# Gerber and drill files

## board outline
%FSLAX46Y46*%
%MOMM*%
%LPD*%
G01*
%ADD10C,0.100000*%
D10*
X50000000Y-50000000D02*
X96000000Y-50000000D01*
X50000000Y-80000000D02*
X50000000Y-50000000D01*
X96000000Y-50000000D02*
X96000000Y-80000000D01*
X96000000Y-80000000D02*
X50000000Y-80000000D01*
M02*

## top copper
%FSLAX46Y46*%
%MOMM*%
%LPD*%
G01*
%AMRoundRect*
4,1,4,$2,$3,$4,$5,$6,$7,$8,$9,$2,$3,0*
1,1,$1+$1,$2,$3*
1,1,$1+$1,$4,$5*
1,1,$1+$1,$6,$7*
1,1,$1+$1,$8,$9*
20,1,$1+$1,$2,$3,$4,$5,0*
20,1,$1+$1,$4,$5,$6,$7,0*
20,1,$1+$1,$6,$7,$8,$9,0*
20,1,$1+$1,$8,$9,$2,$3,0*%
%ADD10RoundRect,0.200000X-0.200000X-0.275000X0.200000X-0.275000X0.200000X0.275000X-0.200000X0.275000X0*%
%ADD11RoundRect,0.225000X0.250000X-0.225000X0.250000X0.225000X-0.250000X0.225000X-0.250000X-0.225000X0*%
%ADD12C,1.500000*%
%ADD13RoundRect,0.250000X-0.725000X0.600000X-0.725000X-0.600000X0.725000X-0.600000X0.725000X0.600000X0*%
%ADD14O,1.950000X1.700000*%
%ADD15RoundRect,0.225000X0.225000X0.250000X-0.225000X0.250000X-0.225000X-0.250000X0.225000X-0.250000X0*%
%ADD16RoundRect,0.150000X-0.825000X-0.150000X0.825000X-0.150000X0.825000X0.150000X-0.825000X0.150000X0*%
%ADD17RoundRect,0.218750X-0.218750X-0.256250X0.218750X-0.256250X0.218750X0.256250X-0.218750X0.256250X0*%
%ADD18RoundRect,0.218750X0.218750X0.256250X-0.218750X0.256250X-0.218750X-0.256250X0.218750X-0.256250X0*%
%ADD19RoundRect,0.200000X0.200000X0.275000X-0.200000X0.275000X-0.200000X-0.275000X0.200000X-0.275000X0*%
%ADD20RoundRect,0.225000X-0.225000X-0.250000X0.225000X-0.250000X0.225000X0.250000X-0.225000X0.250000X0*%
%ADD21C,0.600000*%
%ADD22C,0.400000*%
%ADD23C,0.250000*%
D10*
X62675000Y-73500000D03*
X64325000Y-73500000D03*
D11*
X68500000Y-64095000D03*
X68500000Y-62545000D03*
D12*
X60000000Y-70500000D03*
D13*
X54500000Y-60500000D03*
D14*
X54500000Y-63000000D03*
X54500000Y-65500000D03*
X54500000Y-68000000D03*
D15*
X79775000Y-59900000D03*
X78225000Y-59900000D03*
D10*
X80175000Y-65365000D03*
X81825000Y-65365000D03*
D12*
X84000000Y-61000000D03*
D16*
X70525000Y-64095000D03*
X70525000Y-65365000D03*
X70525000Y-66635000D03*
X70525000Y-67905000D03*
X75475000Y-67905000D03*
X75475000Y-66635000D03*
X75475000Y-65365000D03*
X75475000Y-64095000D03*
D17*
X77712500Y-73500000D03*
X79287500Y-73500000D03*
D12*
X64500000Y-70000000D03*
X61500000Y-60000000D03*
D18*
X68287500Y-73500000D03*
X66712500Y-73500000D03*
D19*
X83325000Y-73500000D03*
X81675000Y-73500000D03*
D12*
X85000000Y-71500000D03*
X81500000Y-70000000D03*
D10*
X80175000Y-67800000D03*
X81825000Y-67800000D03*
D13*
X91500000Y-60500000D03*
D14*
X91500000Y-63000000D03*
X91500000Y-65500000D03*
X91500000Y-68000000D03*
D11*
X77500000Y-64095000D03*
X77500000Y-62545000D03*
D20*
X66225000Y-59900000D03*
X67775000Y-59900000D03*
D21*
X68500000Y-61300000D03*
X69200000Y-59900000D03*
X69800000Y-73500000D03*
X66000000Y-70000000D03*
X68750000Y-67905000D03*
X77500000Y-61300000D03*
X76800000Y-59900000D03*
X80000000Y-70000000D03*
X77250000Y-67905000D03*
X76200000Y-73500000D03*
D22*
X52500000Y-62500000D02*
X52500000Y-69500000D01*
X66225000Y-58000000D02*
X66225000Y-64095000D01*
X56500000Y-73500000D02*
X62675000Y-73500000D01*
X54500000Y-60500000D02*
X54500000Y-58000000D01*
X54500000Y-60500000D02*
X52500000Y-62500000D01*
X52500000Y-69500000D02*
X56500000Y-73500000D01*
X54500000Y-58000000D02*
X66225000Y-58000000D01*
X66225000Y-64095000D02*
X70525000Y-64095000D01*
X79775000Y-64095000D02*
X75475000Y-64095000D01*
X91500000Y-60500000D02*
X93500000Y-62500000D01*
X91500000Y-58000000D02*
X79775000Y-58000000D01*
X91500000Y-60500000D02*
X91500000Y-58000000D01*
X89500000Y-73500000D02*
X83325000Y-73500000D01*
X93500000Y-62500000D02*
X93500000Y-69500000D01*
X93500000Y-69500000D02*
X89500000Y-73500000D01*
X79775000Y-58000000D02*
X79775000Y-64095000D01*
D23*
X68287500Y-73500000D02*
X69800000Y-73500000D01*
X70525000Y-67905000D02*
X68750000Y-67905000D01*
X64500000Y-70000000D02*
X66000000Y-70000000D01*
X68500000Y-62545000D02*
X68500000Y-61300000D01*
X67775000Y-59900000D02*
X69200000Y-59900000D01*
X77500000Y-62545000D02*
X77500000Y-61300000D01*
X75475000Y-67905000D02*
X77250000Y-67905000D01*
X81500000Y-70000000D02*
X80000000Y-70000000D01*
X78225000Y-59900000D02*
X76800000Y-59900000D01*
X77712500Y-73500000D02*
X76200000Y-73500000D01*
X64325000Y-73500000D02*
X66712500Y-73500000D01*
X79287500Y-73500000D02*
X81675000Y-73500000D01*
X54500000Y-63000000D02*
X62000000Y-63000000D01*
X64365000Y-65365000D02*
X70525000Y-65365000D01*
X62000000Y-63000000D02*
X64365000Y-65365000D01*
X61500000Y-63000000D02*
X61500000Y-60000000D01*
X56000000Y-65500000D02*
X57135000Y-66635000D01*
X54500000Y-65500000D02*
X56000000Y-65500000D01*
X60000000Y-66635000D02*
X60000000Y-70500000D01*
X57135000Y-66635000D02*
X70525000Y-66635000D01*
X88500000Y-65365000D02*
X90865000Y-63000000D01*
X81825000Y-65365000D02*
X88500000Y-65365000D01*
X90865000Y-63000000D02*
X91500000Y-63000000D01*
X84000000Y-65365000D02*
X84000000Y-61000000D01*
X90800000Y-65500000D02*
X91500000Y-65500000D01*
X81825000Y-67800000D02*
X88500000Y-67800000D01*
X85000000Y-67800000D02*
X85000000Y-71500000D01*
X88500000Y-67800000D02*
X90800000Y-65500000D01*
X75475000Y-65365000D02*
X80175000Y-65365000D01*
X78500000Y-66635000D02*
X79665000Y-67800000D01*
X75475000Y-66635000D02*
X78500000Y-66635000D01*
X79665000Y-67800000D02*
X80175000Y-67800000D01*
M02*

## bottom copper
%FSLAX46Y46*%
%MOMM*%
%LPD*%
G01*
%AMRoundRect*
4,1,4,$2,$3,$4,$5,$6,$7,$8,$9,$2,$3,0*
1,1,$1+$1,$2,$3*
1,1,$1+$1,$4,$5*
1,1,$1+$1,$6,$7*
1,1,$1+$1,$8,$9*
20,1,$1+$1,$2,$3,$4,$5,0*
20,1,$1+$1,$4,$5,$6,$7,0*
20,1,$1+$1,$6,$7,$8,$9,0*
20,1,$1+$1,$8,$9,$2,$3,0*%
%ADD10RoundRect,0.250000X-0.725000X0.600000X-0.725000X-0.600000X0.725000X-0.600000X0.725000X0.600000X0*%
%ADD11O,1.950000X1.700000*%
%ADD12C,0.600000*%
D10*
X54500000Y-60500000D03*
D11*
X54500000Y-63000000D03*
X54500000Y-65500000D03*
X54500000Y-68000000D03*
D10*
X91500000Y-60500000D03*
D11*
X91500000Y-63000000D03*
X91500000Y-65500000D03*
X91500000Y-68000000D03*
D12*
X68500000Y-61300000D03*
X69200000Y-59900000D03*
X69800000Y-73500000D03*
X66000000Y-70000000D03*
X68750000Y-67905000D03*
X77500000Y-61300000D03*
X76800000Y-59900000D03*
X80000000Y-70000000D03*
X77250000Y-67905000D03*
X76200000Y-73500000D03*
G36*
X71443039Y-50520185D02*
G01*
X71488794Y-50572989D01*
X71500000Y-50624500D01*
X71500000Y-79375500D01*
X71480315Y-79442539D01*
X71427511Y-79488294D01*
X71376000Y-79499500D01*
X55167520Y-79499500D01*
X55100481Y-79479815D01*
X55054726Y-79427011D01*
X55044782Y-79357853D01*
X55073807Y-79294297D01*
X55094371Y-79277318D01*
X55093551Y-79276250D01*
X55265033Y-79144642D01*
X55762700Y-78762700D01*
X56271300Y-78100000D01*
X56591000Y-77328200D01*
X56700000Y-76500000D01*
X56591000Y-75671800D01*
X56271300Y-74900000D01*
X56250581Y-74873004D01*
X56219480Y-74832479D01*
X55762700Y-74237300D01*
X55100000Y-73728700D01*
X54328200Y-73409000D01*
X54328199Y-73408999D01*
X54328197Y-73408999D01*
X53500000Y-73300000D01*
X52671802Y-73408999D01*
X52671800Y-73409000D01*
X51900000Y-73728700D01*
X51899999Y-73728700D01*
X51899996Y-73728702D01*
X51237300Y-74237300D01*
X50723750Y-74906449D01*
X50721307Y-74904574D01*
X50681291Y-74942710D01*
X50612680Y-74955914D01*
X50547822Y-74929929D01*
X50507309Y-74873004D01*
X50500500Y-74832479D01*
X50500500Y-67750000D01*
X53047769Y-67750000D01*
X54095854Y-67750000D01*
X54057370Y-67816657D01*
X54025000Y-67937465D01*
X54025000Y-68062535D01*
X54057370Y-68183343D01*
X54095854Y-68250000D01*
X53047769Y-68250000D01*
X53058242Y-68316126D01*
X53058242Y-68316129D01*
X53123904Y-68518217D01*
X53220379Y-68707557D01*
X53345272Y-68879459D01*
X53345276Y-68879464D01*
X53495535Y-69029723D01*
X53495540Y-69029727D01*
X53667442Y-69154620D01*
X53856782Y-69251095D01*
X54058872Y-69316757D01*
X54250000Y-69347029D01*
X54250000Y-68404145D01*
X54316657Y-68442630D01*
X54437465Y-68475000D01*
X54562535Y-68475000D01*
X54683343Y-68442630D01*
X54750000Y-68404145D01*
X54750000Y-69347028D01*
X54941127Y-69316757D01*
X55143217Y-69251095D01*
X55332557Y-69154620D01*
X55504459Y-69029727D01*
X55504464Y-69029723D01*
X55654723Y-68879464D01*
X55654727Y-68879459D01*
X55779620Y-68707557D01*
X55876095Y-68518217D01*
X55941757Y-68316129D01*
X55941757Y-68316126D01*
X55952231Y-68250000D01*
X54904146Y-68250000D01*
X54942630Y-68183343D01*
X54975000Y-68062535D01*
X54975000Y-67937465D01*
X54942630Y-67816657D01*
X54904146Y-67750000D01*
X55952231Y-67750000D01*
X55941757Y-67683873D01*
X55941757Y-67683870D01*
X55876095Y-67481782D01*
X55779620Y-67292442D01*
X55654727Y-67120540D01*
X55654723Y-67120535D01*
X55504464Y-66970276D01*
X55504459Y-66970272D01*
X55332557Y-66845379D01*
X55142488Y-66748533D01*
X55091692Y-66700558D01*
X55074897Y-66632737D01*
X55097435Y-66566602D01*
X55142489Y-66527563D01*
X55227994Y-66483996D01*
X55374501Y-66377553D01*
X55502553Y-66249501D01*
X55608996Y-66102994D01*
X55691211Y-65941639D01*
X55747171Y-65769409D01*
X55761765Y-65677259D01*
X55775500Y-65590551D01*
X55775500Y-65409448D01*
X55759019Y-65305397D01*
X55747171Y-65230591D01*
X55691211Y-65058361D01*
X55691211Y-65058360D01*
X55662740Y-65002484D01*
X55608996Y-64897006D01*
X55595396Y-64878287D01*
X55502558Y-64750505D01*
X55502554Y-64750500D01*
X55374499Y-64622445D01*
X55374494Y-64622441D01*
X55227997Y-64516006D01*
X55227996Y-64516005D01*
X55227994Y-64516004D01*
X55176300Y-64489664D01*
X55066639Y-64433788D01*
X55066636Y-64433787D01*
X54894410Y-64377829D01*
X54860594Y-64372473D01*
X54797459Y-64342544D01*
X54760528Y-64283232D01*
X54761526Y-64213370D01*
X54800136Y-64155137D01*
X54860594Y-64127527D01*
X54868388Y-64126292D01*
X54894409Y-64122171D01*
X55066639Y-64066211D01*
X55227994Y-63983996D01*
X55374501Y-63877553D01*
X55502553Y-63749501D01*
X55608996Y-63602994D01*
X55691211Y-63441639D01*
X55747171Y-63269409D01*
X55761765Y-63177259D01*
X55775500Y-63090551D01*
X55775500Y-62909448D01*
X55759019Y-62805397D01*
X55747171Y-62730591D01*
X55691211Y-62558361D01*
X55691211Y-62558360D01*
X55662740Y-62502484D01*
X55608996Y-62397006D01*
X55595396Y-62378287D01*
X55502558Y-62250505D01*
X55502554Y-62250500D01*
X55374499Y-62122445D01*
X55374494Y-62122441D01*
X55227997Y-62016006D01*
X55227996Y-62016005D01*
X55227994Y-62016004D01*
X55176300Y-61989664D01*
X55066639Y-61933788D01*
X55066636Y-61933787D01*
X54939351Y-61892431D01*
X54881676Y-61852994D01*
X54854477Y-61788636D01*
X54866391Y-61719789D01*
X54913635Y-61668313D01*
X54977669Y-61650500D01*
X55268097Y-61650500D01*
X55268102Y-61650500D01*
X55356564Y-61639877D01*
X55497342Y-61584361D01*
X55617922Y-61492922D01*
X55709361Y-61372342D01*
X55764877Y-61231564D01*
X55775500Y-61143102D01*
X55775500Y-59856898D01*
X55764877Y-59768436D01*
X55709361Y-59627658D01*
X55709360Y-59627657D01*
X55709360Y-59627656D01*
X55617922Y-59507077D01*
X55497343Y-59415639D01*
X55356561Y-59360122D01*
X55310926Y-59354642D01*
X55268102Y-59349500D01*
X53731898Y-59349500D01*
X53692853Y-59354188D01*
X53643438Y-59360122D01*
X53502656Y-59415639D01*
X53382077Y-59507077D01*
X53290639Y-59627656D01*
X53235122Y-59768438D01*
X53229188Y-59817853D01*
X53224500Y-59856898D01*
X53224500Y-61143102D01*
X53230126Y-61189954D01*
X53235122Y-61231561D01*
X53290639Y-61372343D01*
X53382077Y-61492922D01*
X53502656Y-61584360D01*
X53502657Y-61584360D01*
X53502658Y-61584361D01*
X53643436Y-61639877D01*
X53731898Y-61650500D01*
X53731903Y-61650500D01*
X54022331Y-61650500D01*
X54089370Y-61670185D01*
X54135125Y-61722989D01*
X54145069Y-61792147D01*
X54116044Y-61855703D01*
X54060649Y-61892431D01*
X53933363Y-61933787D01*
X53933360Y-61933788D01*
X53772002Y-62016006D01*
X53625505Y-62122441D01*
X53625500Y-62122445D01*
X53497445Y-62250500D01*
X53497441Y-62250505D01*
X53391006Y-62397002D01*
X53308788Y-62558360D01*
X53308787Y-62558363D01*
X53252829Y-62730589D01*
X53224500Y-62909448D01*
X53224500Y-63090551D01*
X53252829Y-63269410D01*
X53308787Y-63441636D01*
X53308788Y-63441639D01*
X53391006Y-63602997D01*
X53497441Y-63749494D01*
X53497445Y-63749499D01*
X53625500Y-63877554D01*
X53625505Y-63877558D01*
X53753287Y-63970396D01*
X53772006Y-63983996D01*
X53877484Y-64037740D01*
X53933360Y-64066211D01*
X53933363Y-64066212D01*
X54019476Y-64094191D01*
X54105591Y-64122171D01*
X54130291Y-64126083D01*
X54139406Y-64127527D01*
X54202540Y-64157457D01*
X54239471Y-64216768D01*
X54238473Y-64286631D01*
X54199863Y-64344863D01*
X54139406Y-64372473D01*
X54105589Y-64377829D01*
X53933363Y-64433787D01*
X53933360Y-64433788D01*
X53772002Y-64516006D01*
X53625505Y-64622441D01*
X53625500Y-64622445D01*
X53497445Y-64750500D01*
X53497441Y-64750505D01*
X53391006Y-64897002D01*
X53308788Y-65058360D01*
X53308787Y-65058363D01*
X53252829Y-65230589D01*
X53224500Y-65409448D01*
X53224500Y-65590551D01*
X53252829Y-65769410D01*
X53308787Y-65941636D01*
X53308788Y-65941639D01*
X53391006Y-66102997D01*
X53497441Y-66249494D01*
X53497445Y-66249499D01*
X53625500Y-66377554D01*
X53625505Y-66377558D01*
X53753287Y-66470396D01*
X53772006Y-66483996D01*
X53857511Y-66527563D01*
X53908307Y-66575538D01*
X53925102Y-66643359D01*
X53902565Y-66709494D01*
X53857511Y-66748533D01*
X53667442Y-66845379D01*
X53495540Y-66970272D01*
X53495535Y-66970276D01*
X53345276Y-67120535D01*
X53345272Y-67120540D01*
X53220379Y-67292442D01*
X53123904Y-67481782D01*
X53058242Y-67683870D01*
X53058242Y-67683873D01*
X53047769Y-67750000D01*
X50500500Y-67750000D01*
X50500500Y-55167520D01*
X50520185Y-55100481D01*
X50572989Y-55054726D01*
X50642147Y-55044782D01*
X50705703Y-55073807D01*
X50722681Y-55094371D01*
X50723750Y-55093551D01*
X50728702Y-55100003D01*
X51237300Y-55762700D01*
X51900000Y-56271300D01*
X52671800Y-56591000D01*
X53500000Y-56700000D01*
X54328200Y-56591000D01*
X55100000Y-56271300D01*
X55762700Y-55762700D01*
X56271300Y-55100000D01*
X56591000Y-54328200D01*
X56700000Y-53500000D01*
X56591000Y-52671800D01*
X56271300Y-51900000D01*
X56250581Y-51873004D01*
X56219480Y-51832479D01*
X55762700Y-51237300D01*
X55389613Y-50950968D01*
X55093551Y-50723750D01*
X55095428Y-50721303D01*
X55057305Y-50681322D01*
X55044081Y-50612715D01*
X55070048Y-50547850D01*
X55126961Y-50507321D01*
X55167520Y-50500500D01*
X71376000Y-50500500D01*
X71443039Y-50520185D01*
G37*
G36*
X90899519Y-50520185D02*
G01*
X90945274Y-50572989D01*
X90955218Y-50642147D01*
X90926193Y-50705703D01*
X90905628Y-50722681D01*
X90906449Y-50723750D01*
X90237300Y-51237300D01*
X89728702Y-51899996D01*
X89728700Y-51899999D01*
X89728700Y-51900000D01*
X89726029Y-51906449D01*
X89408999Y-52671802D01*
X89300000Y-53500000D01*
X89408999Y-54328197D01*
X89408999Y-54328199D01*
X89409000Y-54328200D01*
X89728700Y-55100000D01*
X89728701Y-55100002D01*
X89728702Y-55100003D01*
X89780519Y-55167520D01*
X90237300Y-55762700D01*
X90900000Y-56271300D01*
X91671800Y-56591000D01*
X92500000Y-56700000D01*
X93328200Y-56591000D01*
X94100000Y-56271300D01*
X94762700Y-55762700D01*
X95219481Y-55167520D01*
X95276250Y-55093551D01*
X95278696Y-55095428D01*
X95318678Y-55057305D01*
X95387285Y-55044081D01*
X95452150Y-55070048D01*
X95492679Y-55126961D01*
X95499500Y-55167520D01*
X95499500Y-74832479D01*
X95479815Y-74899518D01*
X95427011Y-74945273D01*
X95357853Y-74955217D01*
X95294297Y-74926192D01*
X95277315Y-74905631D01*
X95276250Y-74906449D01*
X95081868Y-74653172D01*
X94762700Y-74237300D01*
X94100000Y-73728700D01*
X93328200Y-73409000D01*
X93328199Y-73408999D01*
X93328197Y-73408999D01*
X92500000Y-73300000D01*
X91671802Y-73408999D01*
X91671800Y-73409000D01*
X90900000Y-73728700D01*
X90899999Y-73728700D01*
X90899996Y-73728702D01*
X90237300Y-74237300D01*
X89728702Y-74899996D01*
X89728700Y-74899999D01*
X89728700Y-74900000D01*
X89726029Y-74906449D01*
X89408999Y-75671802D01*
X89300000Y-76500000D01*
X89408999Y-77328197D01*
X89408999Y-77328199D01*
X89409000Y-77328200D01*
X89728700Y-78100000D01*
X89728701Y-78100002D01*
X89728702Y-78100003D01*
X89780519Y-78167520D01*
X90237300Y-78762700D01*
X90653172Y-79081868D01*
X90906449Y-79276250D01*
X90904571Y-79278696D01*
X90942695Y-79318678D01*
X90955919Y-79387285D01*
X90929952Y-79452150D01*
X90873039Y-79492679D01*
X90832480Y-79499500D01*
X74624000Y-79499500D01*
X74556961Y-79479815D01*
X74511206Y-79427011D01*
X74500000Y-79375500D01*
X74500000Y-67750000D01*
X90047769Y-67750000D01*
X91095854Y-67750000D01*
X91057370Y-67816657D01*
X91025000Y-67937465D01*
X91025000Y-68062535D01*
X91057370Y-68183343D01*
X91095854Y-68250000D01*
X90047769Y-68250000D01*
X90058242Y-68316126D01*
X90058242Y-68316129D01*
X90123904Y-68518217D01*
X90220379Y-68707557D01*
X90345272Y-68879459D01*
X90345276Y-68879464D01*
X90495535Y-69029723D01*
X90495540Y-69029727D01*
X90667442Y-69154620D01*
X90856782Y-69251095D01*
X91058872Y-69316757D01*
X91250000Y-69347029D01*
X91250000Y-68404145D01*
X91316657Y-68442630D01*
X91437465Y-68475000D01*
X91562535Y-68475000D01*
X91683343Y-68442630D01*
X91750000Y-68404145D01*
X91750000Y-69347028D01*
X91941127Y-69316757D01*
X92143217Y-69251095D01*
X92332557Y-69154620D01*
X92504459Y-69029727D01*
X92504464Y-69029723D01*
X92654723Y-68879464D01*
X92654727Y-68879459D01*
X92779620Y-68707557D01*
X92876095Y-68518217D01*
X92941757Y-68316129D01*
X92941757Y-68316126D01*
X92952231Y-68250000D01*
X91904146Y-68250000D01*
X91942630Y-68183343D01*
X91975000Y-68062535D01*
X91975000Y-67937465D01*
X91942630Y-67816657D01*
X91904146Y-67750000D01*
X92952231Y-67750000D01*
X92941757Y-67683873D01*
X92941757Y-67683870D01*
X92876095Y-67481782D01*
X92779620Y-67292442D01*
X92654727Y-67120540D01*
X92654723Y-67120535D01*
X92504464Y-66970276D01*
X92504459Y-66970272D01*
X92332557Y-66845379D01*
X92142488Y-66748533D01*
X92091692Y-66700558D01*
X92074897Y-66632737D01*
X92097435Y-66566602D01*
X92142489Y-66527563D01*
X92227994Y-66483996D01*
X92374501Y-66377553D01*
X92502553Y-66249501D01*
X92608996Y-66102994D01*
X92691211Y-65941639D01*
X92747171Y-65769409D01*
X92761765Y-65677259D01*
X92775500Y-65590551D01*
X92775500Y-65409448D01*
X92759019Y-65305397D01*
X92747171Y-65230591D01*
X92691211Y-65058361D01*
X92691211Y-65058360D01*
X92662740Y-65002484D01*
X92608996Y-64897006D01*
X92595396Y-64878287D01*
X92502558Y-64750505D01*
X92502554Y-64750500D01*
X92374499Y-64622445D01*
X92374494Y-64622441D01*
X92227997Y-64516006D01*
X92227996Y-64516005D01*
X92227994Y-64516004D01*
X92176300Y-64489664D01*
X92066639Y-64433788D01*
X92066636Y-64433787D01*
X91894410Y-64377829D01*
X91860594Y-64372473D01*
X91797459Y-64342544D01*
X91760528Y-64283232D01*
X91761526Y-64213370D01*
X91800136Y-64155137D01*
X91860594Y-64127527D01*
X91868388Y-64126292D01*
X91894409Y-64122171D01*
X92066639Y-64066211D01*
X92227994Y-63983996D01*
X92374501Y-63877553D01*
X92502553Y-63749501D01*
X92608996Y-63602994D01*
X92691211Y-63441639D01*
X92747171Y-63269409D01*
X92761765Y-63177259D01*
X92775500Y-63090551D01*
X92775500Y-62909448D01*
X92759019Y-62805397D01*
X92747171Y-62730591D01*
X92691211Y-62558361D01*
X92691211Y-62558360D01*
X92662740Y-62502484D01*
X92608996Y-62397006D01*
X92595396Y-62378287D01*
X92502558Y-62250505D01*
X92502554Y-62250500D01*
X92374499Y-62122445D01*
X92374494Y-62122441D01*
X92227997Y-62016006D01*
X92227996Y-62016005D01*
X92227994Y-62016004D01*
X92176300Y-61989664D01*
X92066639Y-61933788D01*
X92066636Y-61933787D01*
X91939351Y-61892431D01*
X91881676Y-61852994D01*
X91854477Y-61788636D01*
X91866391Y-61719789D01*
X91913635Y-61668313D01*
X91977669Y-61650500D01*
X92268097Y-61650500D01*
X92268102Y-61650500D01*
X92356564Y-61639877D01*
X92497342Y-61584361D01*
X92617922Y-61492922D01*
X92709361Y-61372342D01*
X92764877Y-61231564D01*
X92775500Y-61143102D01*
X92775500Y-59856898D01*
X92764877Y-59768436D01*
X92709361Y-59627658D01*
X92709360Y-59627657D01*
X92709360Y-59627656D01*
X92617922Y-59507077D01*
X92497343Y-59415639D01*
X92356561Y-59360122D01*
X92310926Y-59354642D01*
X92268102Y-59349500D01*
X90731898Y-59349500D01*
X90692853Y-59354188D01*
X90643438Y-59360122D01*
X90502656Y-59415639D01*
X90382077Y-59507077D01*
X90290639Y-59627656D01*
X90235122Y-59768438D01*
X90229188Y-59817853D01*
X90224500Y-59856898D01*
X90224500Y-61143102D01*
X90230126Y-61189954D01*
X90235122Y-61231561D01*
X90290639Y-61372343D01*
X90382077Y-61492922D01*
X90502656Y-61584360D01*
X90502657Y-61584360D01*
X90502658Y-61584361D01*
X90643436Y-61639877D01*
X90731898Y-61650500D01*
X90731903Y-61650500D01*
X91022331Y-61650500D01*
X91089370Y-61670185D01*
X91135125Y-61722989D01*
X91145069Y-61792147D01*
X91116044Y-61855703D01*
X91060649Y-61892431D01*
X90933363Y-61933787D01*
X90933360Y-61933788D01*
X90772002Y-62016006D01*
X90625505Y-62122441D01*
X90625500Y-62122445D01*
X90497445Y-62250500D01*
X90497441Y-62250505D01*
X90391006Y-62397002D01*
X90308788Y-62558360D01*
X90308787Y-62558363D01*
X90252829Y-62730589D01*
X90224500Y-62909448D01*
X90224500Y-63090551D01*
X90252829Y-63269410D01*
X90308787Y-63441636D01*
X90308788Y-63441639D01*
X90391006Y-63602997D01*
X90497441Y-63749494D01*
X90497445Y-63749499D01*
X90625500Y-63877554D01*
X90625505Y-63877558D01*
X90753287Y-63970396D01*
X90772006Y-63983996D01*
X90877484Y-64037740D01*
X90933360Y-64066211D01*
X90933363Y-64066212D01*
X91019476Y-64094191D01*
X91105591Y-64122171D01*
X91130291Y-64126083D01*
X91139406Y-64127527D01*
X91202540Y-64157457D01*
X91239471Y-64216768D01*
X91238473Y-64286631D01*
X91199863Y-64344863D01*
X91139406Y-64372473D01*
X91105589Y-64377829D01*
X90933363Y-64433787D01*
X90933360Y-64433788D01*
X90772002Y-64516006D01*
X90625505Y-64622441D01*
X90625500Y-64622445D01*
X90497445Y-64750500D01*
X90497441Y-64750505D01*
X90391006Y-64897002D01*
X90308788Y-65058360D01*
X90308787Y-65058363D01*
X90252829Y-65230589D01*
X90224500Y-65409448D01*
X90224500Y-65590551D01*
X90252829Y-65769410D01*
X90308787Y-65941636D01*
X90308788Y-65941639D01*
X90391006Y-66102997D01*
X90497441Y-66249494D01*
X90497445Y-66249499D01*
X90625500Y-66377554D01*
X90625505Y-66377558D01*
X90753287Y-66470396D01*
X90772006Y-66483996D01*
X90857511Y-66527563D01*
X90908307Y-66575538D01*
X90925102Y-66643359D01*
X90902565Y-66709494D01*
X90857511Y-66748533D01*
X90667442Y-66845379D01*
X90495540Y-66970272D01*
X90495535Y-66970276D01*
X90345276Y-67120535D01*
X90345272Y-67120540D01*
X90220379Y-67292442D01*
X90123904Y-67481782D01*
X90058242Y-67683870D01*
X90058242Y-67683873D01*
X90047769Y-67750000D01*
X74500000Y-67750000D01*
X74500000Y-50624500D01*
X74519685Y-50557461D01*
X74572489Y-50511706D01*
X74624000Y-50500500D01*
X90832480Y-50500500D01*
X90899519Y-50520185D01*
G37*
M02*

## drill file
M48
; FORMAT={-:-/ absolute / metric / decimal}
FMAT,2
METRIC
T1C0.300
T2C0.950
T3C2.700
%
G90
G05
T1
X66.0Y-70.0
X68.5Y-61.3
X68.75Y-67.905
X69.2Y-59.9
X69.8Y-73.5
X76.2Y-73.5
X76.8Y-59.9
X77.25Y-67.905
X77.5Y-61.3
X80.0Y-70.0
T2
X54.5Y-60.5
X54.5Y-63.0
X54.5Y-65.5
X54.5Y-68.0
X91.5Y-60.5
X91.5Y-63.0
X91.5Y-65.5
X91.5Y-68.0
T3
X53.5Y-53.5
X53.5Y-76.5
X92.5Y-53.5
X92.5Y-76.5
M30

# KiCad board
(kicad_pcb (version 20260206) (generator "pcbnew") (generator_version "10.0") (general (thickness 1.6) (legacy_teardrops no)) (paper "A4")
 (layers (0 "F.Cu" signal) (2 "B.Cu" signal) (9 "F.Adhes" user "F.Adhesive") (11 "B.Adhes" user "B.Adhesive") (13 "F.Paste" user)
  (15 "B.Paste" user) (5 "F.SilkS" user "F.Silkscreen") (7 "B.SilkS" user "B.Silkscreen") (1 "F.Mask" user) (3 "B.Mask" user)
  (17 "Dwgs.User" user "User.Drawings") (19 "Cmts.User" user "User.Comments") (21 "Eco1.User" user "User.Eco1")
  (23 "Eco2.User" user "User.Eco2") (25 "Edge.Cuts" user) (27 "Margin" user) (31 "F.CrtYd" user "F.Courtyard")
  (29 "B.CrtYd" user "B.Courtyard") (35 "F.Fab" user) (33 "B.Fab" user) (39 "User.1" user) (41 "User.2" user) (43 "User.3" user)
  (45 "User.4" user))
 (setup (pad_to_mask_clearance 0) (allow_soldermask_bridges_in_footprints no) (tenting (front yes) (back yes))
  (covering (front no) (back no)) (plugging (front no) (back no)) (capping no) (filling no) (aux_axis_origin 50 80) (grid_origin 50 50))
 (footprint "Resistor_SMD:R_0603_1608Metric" (layer "F.Cu") (at 63.5 73.5)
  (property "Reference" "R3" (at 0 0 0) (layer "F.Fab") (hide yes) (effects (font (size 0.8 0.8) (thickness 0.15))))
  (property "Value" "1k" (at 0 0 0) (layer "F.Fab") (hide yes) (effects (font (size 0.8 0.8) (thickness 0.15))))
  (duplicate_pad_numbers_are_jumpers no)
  (pad "1" smd roundrect (at -0.825 0) (size 0.8 0.95) (layers "F.Cu" "F.Mask" "F.Paste") (roundrect_rratio 0.25) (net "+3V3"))
  (pad "2" smd roundrect (at 0.825 0) (size 0.8 0.95) (layers "F.Cu" "F.Mask" "F.Paste") (roundrect_rratio 0.25) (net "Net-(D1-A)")))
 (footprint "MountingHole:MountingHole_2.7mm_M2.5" (layer "F.Cu") (at 92.5 53.5)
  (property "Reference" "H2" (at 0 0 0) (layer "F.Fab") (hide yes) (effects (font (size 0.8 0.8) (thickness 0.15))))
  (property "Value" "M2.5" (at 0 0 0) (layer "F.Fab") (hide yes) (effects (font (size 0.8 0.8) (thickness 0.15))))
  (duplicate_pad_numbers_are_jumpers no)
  (pad "" np_thru_hole circle (at 0 0) (size 2.7 2.7) (drill 2.7) (layers "*.Cu" "*.Mask")))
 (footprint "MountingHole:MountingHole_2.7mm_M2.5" (layer "F.Cu") (at 92.5 76.5)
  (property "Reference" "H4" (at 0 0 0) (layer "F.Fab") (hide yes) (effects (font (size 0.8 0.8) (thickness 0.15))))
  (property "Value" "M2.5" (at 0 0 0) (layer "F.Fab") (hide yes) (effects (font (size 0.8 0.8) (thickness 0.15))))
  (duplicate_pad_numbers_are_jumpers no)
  (pad "" np_thru_hole circle (at 0 0) (size 2.7 2.7) (drill 2.7) (layers "*.Cu" "*.Mask")))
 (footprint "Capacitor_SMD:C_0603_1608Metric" (layer "F.Cu") (at 68.5 63.32 90)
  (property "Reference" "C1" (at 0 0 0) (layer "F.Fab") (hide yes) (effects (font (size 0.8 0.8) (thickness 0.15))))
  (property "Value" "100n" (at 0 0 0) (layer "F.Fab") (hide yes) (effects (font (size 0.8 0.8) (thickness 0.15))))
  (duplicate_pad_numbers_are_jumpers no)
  (pad "1" smd roundrect (at -0.775 0 90) (size 0.9 0.95) (layers "F.Cu" "F.Mask" "F.Paste") (roundrect_rratio 0.25) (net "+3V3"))
  (pad "2" smd roundrect (at 0.775 0 90) (size 0.9 0.95) (layers "F.Cu" "F.Mask" "F.Paste") (roundrect_rratio 0.25) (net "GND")))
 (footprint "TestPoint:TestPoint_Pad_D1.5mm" (layer "F.Cu") (at 60 70.5)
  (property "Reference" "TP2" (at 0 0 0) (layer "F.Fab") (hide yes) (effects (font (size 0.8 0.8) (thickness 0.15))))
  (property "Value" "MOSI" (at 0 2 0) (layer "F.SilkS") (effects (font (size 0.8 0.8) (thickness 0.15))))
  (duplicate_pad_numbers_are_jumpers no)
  (pad "1" smd circle (at 0 0) (size 1.5 1.5) (layers "F.Cu" "F.Mask") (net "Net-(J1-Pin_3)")))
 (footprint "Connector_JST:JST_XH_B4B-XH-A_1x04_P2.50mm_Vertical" (layer "F.Cu") (at 54.5 60.5 -90)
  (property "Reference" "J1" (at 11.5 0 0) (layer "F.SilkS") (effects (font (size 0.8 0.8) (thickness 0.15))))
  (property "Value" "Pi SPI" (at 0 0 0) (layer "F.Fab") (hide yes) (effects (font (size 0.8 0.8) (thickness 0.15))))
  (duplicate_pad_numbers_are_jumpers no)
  (pad "1" thru_hole roundrect (at 0 0 270) (size 1.7 1.95) (drill 0.95) (layers "*.Cu" "*.Mask") (remove_unused_layers no)
   (roundrect_rratio 0.147059) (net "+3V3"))
  (pad "2" thru_hole oval (at 2.5 0 270) (size 1.7 1.95) (drill 0.95) (layers "*.Cu" "*.Mask") (remove_unused_layers no)
   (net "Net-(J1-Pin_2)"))
  (pad "3" thru_hole oval (at 5 0 270) (size 1.7 1.95) (drill 0.95) (layers "*.Cu" "*.Mask") (remove_unused_layers no)
   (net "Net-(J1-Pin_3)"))
  (pad "4" thru_hole oval (at 7.5 0 270) (size 1.7 1.95) (drill 0.95) (layers "*.Cu" "*.Mask") (remove_unused_layers no) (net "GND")))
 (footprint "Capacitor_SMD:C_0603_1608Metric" (layer "F.Cu") (at 79 59.9 180)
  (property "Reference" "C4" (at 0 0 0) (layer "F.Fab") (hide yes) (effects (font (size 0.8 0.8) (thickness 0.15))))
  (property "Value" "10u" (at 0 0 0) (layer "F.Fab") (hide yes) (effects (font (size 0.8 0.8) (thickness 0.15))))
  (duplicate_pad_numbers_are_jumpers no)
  (pad "1" smd roundrect (at -0.775 0 180) (size 0.9 0.95) (layers "F.Cu" "F.Mask" "F.Paste") (roundrect_rratio 0.25) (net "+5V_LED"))
  (pad "2" smd roundrect (at 0.775 0 180) (size 0.9 0.95) (layers "F.Cu" "F.Mask" "F.Paste") (roundrect_rratio 0.25) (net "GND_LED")))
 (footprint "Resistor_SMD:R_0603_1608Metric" (layer "F.Cu") (at 81 65.365)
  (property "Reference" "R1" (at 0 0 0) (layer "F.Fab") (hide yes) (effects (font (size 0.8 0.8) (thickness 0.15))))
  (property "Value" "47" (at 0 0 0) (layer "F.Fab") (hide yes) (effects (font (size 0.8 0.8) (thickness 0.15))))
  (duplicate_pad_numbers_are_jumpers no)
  (pad "1" smd roundrect (at -0.825 0) (size 0.8 0.95) (layers "F.Cu" "F.Mask" "F.Paste") (roundrect_rratio 0.25) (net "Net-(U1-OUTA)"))
  (pad "2" smd roundrect (at 0.825 0) (size 0.8 0.95) (layers "F.Cu" "F.Mask" "F.Paste") (roundrect_rratio 0.25) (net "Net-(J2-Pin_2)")))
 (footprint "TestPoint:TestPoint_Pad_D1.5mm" (layer "F.Cu") (at 84 61)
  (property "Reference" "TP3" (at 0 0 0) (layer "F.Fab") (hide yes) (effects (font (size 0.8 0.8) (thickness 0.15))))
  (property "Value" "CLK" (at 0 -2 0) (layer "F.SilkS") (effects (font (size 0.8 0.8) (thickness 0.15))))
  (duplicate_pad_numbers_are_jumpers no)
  (pad "1" smd circle (at 0 0) (size 1.5 1.5) (layers "F.Cu" "F.Mask") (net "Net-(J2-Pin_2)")))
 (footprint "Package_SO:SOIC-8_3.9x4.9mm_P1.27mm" (layer "F.Cu") (at 73 66)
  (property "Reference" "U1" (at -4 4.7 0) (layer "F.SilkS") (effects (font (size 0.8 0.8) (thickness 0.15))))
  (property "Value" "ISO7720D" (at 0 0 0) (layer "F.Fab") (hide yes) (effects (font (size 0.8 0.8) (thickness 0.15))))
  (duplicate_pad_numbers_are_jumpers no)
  (pad "1" smd roundrect (at -2.475 -1.905) (size 1.95 0.6) (layers "F.Cu" "F.Mask" "F.Paste") (roundrect_rratio 0.25) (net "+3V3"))
  (pad "2" smd roundrect (at -2.475 -0.635) (size 1.95 0.6) (layers "F.Cu" "F.Mask" "F.Paste") (roundrect_rratio 0.25)
   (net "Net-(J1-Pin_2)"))
  (pad "3" smd roundrect (at -2.475 0.635) (size 1.95 0.6) (layers "F.Cu" "F.Mask" "F.Paste") (roundrect_rratio 0.25) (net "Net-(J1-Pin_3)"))
  (pad "4" smd roundrect (at -2.475 1.905) (size 1.95 0.6) (layers "F.Cu" "F.Mask" "F.Paste") (roundrect_rratio 0.25) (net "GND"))
  (pad "5" smd roundrect (at 2.475 1.905) (size 1.95 0.6) (layers "F.Cu" "F.Mask" "F.Paste") (roundrect_rratio 0.25) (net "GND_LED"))
  (pad "6" smd roundrect (at 2.475 0.635) (size 1.95 0.6) (layers "F.Cu" "F.Mask" "F.Paste") (roundrect_rratio 0.25) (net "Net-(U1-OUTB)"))
  (pad "7" smd roundrect (at 2.475 -0.635) (size 1.95 0.6) (layers "F.Cu" "F.Mask" "F.Paste") (roundrect_rratio 0.25) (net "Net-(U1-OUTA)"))
  (pad "8" smd roundrect (at 2.475 -1.905) (size 1.95 0.6) (layers "F.Cu" "F.Mask" "F.Paste") (roundrect_rratio 0.25) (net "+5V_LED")))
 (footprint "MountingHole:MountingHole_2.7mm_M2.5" (layer "F.Cu") (at 53.5 53.5)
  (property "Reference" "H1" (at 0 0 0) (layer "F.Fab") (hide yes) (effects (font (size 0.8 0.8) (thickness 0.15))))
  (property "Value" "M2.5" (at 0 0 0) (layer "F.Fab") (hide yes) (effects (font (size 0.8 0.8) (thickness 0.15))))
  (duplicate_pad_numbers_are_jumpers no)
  (pad "" np_thru_hole circle (at 0 0) (size 2.7 2.7) (drill 2.7) (layers "*.Cu" "*.Mask")))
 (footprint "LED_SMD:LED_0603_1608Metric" (layer "F.Cu") (at 78.5 73.5)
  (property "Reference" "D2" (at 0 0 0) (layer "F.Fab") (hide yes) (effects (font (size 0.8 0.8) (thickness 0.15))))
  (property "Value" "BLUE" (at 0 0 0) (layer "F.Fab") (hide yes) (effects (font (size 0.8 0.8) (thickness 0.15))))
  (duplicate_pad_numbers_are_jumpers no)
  (pad "1" smd roundrect (at -0.7875 0) (size 0.875 0.95) (layers "F.Cu" "F.Mask" "F.Paste") (roundrect_rratio 0.25) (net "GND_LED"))
  (pad "2" smd roundrect (at 0.7875 0) (size 0.875 0.95) (layers "F.Cu" "F.Mask" "F.Paste") (roundrect_rratio 0.25) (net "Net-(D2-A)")))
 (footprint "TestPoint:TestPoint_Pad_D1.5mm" (layer "F.Cu") (at 64.5 70)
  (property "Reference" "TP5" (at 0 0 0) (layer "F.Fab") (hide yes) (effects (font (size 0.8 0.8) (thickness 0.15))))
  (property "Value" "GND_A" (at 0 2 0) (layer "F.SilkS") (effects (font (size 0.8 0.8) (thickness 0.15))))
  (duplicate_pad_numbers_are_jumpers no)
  (pad "1" smd circle (at 0 0) (size 1.5 1.5) (layers "F.Cu" "F.Mask") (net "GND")))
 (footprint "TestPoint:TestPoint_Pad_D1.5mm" (layer "F.Cu") (at 61.5 60)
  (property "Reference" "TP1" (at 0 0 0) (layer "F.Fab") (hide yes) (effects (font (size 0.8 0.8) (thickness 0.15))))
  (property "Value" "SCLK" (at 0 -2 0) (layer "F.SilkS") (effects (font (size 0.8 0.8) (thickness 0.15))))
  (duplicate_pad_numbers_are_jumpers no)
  (pad "1" smd circle (at 0 0) (size 1.5 1.5) (layers "F.Cu" "F.Mask") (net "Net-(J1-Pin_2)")))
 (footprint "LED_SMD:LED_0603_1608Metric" (layer "F.Cu") (at 67.5 73.5 180)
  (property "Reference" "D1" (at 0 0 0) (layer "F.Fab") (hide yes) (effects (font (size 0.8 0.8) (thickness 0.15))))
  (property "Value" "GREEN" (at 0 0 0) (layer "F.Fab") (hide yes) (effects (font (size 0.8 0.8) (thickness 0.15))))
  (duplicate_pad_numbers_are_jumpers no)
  (pad "1" smd roundrect (at -0.7875 0 180) (size 0.875 0.95) (layers "F.Cu" "F.Mask" "F.Paste") (roundrect_rratio 0.25) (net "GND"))
  (pad "2" smd roundrect (at 0.7875 0 180) (size 0.875 0.95) (layers "F.Cu" "F.Mask" "F.Paste") (roundrect_rratio 0.25) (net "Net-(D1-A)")))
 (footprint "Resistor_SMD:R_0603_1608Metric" (layer "F.Cu") (at 82.5 73.5 180)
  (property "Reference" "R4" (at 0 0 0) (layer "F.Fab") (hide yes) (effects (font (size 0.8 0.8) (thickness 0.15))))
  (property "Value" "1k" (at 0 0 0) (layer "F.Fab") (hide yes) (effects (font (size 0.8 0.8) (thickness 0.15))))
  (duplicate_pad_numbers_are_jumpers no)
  (pad "1" smd roundrect (at -0.825 0 180) (size 0.8 0.95) (layers "F.Cu" "F.Mask" "F.Paste") (roundrect_rratio 0.25) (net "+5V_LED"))
  (pad "2" smd roundrect (at 0.825 0 180) (size 0.8 0.95) (layers "F.Cu" "F.Mask" "F.Paste") (roundrect_rratio 0.25) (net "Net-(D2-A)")))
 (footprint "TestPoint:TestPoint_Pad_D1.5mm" (layer "F.Cu") (at 85 71.5)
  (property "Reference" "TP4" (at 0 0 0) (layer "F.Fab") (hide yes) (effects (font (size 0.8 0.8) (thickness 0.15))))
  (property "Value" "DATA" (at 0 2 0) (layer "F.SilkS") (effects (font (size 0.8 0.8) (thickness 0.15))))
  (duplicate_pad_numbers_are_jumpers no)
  (pad "1" smd circle (at 0 0) (size 1.5 1.5) (layers "F.Cu" "F.Mask") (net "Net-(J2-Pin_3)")))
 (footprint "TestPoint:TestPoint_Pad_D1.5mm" (layer "F.Cu") (at 81.5 70)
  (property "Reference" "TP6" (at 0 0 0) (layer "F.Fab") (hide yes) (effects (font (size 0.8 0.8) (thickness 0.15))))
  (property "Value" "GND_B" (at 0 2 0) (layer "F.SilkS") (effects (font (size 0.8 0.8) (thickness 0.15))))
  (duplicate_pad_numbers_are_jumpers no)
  (pad "1" smd circle (at 0 0) (size 1.5 1.5) (layers "F.Cu" "F.Mask") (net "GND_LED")))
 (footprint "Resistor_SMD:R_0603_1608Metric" (layer "F.Cu") (at 81 67.8)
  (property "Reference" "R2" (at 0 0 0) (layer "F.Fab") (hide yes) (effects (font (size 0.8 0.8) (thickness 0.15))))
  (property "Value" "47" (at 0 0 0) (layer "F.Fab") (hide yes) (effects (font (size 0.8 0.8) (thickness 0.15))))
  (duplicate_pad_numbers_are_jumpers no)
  (pad "1" smd roundrect (at -0.825 0) (size 0.8 0.95) (layers "F.Cu" "F.Mask" "F.Paste") (roundrect_rratio 0.25) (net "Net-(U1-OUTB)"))
  (pad "2" smd roundrect (at 0.825 0) (size 0.8 0.95) (layers "F.Cu" "F.Mask" "F.Paste") (roundrect_rratio 0.25) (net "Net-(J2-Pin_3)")))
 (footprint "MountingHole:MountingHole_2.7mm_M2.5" (layer "F.Cu") (at 53.5 76.5)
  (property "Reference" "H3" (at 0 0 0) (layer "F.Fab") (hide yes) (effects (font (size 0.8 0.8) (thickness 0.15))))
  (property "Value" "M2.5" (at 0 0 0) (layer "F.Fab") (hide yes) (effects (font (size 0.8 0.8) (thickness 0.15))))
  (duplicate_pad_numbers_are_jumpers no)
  (pad "" np_thru_hole circle (at 0 0) (size 2.7 2.7) (drill 2.7) (layers "*.Cu" "*.Mask")))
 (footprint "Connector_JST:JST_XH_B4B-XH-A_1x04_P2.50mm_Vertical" (layer "F.Cu") (at 91.5 60.5 -90)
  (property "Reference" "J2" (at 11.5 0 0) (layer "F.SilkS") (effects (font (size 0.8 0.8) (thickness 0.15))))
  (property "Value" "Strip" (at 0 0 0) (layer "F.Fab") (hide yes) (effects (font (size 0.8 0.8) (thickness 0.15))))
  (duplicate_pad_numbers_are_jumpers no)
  (pad "1" thru_hole roundrect (at 0 0 270) (size 1.7 1.95) (drill 0.95) (layers "*.Cu" "*.Mask") (remove_unused_layers no)
   (roundrect_rratio 0.147059) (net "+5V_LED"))
  (pad "2" thru_hole oval (at 2.5 0 270) (size 1.7 1.95) (drill 0.95) (layers "*.Cu" "*.Mask") (remove_unused_layers no)
   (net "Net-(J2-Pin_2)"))
  (pad "3" thru_hole oval (at 5 0 270) (size 1.7 1.95) (drill 0.95) (layers "*.Cu" "*.Mask") (remove_unused_layers no)
   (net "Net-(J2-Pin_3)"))
  (pad "4" thru_hole oval (at 7.5 0 270) (size 1.7 1.95) (drill 0.95) (layers "*.Cu" "*.Mask") (remove_unused_layers no) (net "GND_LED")))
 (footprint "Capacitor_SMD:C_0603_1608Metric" (layer "F.Cu") (at 77.5 63.32 90)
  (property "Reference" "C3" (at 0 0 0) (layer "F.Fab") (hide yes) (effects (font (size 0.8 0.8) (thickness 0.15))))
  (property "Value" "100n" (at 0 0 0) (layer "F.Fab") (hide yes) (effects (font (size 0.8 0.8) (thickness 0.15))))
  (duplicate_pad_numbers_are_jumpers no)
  (pad "1" smd roundrect (at -0.775 0 90) (size 0.9 0.95) (layers "F.Cu" "F.Mask" "F.Paste") (roundrect_rratio 0.25) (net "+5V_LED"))
  (pad "2" smd roundrect (at 0.775 0 90) (size 0.9 0.95) (layers "F.Cu" "F.Mask" "F.Paste") (roundrect_rratio 0.25) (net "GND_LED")))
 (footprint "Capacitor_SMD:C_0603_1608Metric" (layer "F.Cu") (at 67 59.9)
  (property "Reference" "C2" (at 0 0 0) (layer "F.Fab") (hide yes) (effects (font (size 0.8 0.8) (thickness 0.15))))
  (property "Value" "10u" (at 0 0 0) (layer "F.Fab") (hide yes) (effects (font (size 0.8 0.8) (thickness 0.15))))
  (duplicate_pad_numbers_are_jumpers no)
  (pad "1" smd roundrect (at -0.775 0) (size 0.9 0.95) (layers "F.Cu" "F.Mask" "F.Paste") (roundrect_rratio 0.25) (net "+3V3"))
  (pad "2" smd roundrect (at 0.775 0) (size 0.9 0.95) (layers "F.Cu" "F.Mask" "F.Paste") (roundrect_rratio 0.25) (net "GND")))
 (gr_line (start 50 50) (end 96 50) (stroke (width 0.1) (type default)) (layer "Edge.Cuts"))
 (gr_line (start 50 80) (end 50 50) (stroke (width 0.1) (type default)) (layer "Edge.Cuts"))
 (gr_line (start 96 50) (end 96 80) (stroke (width 0.1) (type default)) (layer "Edge.Cuts"))
 (gr_line (start 96 80) (end 50 80) (stroke (width 0.1) (type default)) (layer "Edge.Cuts"))
 (segment (start 52.5 62.5) (end 52.5 69.5) (width 0.4) (layer "F.Cu") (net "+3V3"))
 (segment (start 66.225 58) (end 66.225 64.095) (width 0.4) (layer "F.Cu") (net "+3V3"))
 (segment (start 56.5 73.5) (end 62.675 73.5) (width 0.4) (layer "F.Cu") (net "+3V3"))
 (segment (start 54.5 60.5) (end 54.5 58) (width 0.4) (layer "F.Cu") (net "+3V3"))
 (segment (start 54.5 60.5) (end 52.5 62.5) (width 0.4) (layer "F.Cu") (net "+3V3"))
 (segment (start 52.5 69.5) (end 56.5 73.5) (width 0.4) (layer "F.Cu") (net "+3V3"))
 (segment (start 54.5 58) (end 66.225 58) (width 0.4) (layer "F.Cu") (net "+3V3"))
 (segment (start 66.225 64.095) (end 70.525 64.095) (width 0.4) (layer "F.Cu") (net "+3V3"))
 (segment (start 79.775 64.095) (end 75.475 64.095) (width 0.4) (layer "F.Cu") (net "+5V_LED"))
 (segment (start 91.5 60.5) (end 93.5 62.5) (width 0.4) (layer "F.Cu") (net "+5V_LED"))
 (segment (start 91.5 58) (end 79.775 58) (width 0.4) (layer "F.Cu") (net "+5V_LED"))
 (segment (start 91.5 60.5) (end 91.5 58) (width 0.4) (layer "F.Cu") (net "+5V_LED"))
 (segment (start 89.5 73.5) (end 83.325 73.5) (width 0.4) (layer "F.Cu") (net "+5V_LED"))
 (segment (start 93.5 62.5) (end 93.5 69.5) (width 0.4) (layer "F.Cu") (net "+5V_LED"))
 (segment (start 93.5 69.5) (end 89.5 73.5) (width 0.4) (layer "F.Cu") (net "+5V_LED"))
 (segment (start 79.775 58) (end 79.775 64.095) (width 0.4) (layer "F.Cu") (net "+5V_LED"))
 (segment (start 68.2875 73.5) (end 69.8 73.5) (width 0.25) (layer "F.Cu") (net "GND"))
 (segment (start 70.525 67.905) (end 68.75 67.905) (width 0.25) (layer "F.Cu") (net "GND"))
 (segment (start 64.5 70) (end 66 70) (width 0.25) (layer "F.Cu") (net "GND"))
 (segment (start 68.5 62.545) (end 68.5 61.3) (width 0.25) (layer "F.Cu") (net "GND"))
 (segment (start 67.775 59.9) (end 69.2 59.9) (width 0.25) (layer "F.Cu") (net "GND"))
 (via (at 68.5 61.3) (size 0.6) (drill 0.3) (layers "F.Cu" "B.Cu") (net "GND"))
 (via (at 69.2 59.9) (size 0.6) (drill 0.3) (layers "F.Cu" "B.Cu") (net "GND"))
 (via (at 69.8 73.5) (size 0.6) (drill 0.3) (layers "F.Cu" "B.Cu") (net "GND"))
 (via (at 66 70) (size 0.6) (drill 0.3) (layers "F.Cu" "B.Cu") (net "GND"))
 (via (at 68.75 67.905) (size 0.6) (drill 0.3) (layers "F.Cu" "B.Cu") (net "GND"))
 (segment (start 77.5 62.545) (end 77.5 61.3) (width 0.25) (layer "F.Cu") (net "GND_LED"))
 (segment (start 75.475 67.905) (end 77.25 67.905) (width 0.25) (layer "F.Cu") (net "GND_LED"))
 (segment (start 81.5 70) (end 80 70) (width 0.25) (layer "F.Cu") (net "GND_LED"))
 (segment (start 78.225 59.9) (end 76.8 59.9) (width 0.25) (layer "F.Cu") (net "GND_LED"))
 (segment (start 77.7125 73.5) (end 76.2 73.5) (width 0.25) (layer "F.Cu") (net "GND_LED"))
 (via (at 77.5 61.3) (size 0.6) (drill 0.3) (layers "F.Cu" "B.Cu") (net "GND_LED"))
 (via (at 76.8 59.9) (size 0.6) (drill 0.3) (layers "F.Cu" "B.Cu") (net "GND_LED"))
 (via (at 80 70) (size 0.6) (drill 0.3) (layers "F.Cu" "B.Cu") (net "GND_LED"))
 (via (at 77.25 67.905) (size 0.6) (drill 0.3) (layers "F.Cu" "B.Cu") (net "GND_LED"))
 (via (at 76.2 73.5) (size 0.6) (drill 0.3) (layers "F.Cu" "B.Cu") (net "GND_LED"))
 (segment (start 64.325 73.5) (end 66.7125 73.5) (width 0.25) (layer "F.Cu") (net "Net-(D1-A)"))
 (segment (start 79.2875 73.5) (end 81.675 73.5) (width 0.25) (layer "F.Cu") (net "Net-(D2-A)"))
 (segment (start 54.5 63) (end 62 63) (width 0.25) (layer "F.Cu") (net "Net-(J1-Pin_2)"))
 (segment (start 64.365 65.365) (end 70.525 65.365) (width 0.25) (layer "F.Cu") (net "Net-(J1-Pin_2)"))
 (segment (start 62 63) (end 64.365 65.365) (width 0.25) (layer "F.Cu") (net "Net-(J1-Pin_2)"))
 (segment (start 61.5 63) (end 61.5 60) (width 0.25) (layer "F.Cu") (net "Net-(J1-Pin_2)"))
 (segment (start 56 65.5) (end 57.135 66.635) (width 0.25) (layer "F.Cu") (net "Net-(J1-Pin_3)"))
 (segment (start 54.5 65.5) (end 56 65.5) (width 0.25) (layer "F.Cu") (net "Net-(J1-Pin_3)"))
 (segment (start 60 66.635) (end 60 70.5) (width 0.25) (layer "F.Cu") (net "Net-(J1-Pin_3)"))
 (segment (start 57.135 66.635) (end 70.525 66.635) (width 0.25) (layer "F.Cu") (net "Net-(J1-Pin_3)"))
 (segment (start 88.5 65.365) (end 90.865 63) (width 0.25) (layer "F.Cu") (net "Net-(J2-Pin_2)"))
 (segment (start 81.825 65.365) (end 88.5 65.365) (width 0.25) (layer "F.Cu") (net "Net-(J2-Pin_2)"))
 (segment (start 90.865 63) (end 91.5 63) (width 0.25) (layer "F.Cu") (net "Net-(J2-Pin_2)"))
 (segment (start 84 65.365) (end 84 61) (width 0.25) (layer "F.Cu") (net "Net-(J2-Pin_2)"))
 (segment (start 90.8 65.5) (end 91.5 65.5) (width 0.25) (layer "F.Cu") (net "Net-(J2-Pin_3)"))
 (segment (start 81.825 67.8) (end 88.5 67.8) (width 0.25) (layer "F.Cu") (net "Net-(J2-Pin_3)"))
 (segment (start 85 67.8) (end 85 71.5) (width 0.25) (layer "F.Cu") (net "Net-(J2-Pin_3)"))
 (segment (start 88.5 67.8) (end 90.8 65.5) (width 0.25) (layer "F.Cu") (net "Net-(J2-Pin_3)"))
 (segment (start 75.475 65.365) (end 80.175 65.365) (width 0.25) (layer "F.Cu") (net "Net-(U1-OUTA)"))
 (segment (start 78.5 66.635) (end 79.665 67.8) (width 0.25) (layer "F.Cu") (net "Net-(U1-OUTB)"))
 (segment (start 75.475 66.635) (end 78.5 66.635) (width 0.25) (layer "F.Cu") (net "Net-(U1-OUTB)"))
 (segment (start 79.665 67.8) (end 80.175 67.8) (width 0.25) (layer "F.Cu") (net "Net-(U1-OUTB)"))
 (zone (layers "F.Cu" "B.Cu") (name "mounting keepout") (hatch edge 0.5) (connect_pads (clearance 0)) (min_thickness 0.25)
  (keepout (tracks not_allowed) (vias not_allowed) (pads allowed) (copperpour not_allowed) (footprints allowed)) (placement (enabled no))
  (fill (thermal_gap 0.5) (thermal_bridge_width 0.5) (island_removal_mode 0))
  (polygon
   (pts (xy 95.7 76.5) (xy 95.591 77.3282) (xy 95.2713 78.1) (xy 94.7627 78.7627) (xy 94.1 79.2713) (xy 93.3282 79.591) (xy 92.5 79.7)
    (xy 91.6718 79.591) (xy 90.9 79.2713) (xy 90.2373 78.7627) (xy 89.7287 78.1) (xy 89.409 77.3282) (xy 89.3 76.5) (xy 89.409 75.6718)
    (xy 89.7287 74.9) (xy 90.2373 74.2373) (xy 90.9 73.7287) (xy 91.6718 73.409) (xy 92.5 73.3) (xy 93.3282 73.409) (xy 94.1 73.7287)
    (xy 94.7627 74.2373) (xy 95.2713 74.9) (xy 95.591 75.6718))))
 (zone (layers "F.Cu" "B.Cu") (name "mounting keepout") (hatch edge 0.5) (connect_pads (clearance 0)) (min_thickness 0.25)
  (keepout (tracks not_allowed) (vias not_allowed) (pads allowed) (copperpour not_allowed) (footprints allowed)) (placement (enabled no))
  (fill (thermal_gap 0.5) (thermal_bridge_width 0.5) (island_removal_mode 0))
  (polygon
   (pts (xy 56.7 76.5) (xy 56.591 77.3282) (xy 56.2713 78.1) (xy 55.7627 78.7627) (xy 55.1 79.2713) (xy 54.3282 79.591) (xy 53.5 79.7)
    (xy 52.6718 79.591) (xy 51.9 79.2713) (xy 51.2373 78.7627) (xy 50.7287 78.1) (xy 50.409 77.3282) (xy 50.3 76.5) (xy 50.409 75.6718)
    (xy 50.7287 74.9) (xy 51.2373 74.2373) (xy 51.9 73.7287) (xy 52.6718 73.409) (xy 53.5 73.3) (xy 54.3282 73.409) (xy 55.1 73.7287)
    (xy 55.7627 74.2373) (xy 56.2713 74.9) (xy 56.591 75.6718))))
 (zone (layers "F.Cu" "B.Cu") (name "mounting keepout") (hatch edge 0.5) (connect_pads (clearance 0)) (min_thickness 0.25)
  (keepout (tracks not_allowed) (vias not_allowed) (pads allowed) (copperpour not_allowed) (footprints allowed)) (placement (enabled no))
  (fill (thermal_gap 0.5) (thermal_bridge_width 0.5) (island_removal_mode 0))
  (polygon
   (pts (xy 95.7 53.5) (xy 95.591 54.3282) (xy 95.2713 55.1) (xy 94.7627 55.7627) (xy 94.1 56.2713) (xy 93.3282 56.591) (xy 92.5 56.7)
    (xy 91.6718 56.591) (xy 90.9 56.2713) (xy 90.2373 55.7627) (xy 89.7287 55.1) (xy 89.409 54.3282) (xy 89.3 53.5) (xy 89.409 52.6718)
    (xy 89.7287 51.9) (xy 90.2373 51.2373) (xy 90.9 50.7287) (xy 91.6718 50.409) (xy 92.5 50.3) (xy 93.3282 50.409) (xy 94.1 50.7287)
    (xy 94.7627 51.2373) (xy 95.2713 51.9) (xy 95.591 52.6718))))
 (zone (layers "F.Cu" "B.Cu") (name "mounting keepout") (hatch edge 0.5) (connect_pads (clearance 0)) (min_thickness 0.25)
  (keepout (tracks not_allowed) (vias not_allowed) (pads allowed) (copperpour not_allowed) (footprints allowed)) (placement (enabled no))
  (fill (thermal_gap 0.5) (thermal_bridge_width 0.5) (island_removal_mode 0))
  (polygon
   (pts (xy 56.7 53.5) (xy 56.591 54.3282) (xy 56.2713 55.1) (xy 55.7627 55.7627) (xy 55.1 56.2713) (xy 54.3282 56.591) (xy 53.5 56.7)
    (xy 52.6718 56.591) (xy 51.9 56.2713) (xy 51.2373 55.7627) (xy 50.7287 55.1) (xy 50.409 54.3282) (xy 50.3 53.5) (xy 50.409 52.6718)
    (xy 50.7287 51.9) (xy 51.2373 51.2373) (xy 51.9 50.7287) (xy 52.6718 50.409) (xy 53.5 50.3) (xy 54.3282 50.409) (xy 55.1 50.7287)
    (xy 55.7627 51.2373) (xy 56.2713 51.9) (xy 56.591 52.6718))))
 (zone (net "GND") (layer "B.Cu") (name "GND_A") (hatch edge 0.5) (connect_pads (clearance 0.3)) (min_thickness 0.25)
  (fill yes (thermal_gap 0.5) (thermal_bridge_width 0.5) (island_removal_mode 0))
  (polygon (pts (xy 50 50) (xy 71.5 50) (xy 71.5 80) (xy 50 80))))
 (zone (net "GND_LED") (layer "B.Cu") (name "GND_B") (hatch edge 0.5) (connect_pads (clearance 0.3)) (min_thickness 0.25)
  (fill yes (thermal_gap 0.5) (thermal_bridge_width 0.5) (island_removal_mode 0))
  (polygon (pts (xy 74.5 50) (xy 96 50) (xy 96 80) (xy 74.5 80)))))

